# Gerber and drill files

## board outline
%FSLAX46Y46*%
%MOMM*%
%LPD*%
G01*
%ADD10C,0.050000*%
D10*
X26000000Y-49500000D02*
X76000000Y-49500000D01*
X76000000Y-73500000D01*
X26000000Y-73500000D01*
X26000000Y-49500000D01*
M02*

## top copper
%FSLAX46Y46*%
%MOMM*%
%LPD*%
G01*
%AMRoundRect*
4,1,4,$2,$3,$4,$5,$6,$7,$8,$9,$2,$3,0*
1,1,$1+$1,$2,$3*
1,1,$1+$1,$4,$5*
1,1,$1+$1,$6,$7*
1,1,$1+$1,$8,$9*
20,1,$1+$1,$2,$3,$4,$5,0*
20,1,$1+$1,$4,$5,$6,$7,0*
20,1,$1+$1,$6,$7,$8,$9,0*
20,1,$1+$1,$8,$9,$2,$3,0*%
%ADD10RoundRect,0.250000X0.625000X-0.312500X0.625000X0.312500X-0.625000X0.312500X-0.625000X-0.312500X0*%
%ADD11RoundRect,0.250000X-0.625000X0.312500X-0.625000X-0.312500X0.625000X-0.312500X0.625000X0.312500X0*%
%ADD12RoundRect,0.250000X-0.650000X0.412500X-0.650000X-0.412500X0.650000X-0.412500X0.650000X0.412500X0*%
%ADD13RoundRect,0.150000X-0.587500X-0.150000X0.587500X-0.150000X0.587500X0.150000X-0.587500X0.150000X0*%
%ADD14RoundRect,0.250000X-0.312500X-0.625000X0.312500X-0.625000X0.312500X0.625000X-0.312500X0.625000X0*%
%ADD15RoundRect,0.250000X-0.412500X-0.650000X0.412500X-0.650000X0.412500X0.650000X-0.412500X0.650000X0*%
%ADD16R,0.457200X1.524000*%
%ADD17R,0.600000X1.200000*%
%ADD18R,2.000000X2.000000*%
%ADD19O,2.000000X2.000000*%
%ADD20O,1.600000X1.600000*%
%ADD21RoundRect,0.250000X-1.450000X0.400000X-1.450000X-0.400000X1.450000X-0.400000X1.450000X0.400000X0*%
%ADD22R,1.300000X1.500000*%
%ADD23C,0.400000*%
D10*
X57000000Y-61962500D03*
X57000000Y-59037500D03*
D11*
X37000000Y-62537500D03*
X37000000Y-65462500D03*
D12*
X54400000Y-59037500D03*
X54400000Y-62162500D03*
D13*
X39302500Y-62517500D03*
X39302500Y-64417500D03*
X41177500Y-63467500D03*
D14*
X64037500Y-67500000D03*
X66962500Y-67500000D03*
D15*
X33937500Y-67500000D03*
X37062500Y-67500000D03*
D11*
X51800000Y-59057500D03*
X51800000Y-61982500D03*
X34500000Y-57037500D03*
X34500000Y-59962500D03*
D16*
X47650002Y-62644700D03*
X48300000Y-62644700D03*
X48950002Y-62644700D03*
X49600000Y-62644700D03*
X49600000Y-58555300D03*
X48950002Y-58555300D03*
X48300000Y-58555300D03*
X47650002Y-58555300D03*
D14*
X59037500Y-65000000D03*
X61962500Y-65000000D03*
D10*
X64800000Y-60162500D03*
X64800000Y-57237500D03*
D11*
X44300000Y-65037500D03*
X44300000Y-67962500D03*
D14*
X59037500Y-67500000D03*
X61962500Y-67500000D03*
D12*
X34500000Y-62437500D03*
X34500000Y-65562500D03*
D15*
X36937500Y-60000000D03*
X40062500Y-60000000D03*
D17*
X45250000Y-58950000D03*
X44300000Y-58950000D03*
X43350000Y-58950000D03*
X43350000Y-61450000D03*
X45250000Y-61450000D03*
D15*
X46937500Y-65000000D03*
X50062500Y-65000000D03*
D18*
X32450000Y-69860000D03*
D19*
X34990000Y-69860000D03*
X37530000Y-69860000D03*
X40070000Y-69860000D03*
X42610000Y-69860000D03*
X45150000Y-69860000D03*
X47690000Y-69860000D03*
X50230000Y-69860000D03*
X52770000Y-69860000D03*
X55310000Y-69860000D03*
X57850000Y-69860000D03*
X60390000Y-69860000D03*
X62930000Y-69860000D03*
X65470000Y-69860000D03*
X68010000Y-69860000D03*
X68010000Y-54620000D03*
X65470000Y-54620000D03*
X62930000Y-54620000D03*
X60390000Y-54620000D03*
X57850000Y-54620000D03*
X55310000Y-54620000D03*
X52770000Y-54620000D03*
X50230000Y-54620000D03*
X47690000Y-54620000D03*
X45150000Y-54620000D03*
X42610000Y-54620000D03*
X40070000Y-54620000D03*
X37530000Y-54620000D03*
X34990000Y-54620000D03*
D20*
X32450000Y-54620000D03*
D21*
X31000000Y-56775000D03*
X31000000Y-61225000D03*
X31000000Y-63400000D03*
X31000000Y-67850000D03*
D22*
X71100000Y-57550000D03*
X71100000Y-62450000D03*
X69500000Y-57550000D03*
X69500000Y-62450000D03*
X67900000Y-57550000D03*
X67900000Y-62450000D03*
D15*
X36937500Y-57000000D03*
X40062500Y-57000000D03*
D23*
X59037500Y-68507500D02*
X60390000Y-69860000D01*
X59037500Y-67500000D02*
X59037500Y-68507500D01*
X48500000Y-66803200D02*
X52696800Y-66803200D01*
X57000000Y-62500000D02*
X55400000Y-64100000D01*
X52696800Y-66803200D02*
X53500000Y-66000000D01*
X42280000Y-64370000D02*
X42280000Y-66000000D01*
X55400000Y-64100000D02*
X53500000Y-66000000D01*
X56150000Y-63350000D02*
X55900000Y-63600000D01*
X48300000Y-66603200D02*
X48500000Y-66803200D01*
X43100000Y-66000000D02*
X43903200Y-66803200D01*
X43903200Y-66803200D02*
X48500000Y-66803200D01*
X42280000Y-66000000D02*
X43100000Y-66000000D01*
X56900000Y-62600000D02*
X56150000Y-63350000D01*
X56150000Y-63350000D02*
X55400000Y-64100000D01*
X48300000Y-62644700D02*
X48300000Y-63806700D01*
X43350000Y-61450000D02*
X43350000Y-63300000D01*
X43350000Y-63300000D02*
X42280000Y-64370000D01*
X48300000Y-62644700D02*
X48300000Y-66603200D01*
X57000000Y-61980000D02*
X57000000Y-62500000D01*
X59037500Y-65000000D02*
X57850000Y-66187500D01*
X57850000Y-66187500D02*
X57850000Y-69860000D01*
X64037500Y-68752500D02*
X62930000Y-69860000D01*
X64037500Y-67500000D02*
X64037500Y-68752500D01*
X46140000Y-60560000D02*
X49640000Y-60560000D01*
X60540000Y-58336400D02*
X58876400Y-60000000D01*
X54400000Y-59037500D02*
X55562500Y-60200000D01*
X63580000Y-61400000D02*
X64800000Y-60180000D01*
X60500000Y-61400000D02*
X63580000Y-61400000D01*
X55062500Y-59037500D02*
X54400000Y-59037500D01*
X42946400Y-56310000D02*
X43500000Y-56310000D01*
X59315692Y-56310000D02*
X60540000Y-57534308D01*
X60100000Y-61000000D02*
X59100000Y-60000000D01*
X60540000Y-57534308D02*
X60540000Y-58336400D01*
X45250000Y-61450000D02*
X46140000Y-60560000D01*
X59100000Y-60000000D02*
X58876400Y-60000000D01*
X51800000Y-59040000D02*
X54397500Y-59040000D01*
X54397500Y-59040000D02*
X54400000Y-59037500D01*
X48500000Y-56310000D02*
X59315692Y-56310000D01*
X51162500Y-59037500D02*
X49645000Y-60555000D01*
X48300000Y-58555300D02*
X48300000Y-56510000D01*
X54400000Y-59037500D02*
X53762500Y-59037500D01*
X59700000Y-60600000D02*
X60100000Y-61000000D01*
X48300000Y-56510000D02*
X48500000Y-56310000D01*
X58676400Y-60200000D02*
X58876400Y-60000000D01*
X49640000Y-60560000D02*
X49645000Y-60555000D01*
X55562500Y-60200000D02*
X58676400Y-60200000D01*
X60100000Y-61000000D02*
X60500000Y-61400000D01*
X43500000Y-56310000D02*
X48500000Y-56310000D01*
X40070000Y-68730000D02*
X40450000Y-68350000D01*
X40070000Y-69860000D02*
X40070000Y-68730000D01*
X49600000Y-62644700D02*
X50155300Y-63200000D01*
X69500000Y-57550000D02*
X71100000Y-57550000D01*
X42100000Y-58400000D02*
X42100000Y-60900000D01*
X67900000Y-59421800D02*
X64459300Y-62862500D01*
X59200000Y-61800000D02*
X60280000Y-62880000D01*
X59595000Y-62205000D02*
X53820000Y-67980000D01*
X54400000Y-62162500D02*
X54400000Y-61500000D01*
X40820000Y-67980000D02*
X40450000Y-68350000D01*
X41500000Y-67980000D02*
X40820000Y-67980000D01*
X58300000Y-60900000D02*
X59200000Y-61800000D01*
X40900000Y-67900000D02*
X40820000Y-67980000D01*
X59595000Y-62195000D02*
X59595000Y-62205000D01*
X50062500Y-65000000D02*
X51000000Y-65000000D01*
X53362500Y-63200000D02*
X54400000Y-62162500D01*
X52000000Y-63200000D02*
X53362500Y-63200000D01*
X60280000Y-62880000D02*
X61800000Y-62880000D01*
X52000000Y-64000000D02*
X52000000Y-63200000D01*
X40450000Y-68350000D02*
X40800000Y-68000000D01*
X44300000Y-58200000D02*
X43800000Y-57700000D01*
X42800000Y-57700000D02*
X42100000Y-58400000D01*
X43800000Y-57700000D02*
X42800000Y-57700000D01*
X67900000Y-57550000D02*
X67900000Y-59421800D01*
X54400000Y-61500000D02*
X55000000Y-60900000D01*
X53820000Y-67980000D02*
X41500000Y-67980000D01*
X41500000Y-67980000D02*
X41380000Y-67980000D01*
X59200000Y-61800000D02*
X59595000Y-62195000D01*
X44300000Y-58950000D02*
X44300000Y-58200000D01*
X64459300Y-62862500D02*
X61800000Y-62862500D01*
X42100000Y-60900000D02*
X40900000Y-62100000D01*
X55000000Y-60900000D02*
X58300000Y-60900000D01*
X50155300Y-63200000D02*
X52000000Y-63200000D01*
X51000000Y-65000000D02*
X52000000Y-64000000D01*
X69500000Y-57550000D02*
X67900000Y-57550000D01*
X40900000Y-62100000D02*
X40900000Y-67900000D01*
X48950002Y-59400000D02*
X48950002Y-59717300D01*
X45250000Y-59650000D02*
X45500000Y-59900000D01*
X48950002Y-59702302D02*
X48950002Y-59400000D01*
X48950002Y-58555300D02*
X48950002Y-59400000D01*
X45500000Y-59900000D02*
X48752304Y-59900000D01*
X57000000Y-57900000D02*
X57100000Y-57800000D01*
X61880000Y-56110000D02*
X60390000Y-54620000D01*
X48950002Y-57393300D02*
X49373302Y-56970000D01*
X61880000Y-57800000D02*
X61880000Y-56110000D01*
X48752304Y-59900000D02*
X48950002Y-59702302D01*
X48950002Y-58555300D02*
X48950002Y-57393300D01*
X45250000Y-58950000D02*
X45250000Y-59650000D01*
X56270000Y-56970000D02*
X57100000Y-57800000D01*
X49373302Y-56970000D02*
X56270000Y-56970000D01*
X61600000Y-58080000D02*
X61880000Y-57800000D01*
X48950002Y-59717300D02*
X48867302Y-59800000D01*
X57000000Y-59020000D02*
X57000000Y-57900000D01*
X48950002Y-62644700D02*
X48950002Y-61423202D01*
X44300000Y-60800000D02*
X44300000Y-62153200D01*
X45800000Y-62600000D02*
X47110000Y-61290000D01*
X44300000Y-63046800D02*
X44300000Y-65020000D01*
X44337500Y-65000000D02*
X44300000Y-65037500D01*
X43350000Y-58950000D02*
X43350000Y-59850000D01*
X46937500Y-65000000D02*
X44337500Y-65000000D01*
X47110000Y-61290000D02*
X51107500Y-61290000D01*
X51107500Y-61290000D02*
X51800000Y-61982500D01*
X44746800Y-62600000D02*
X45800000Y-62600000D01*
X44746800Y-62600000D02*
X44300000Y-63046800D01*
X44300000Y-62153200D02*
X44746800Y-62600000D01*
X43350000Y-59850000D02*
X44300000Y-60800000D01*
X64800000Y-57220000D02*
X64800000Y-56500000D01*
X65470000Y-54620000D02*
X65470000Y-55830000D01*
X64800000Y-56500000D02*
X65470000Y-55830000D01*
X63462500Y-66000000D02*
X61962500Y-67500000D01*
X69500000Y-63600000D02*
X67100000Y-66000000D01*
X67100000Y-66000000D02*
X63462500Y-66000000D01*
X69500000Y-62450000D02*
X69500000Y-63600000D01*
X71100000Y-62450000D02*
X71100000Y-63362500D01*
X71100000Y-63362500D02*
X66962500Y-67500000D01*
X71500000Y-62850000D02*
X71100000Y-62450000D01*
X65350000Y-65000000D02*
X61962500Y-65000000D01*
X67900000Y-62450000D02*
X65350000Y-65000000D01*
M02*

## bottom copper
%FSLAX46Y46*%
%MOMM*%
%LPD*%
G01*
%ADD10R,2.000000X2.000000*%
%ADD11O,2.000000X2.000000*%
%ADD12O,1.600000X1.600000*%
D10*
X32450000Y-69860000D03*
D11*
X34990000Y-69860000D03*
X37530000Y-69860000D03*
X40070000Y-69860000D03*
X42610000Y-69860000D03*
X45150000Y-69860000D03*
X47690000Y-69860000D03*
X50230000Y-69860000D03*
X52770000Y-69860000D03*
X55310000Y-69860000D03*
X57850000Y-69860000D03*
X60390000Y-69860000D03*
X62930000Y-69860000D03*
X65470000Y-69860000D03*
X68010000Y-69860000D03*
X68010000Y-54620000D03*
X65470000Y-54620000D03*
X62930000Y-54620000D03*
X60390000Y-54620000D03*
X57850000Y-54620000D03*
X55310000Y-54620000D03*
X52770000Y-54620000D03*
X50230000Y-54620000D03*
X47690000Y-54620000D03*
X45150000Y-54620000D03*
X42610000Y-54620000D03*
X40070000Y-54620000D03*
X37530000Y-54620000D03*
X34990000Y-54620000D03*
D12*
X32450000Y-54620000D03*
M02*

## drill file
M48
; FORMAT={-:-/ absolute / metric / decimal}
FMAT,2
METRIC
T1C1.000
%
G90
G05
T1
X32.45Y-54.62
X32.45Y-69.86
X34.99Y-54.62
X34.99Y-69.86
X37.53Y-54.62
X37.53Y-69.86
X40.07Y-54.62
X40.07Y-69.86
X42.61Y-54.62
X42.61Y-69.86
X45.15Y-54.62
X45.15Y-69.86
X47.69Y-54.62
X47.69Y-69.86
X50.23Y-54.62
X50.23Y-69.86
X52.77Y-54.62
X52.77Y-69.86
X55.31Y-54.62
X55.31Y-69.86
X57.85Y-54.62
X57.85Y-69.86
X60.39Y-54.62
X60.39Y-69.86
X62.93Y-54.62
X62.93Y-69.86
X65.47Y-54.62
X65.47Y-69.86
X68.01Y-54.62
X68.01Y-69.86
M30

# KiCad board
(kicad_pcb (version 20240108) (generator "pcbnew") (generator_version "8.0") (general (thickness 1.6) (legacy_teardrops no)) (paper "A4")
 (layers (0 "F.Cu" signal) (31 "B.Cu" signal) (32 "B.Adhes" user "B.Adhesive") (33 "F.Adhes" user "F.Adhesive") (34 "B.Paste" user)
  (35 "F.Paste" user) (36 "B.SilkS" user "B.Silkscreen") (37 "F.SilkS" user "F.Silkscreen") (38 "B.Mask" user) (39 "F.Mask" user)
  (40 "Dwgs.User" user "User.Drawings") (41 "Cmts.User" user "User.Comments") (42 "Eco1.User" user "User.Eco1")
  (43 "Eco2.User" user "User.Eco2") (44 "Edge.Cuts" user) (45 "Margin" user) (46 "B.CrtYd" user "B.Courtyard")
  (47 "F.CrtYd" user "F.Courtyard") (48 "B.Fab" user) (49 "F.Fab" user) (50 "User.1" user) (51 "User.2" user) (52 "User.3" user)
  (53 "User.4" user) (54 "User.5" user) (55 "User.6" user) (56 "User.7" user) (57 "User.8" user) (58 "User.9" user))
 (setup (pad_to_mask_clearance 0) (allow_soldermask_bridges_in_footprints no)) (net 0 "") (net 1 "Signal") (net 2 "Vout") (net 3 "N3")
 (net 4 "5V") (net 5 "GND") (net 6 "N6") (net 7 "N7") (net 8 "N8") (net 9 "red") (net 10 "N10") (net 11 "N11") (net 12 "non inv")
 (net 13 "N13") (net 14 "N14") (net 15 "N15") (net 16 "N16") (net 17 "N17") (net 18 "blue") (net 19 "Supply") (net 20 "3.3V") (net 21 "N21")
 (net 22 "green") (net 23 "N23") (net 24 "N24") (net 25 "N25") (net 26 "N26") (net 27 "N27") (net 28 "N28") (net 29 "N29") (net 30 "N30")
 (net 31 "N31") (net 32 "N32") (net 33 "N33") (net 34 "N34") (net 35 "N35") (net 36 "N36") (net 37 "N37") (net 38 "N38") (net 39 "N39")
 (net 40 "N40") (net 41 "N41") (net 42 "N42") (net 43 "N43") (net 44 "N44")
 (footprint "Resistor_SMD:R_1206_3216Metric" (layer "F.Cu") (at 57 60.5 90)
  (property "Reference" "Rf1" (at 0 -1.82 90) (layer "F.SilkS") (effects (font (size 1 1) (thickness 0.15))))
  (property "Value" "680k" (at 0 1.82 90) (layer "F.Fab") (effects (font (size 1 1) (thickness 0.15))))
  (pad "1" smd roundrect (at -1.4625 0 90) (size 1.125 1.75) (layers "F.Cu" "F.Paste" "F.Mask") (roundrect_rratio 0.222222) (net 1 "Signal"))
  (pad "2" smd roundrect (at 1.4625 0 90) (size 1.125 1.75) (layers "F.Cu" "F.Paste" "F.Mask") (roundrect_rratio 0.222222) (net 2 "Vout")))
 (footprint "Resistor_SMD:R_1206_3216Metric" (layer "F.Cu") (at 37 64 -90)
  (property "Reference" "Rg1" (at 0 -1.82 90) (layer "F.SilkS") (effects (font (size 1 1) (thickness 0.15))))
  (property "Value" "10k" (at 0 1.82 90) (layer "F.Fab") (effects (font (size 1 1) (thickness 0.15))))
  (pad "1" smd roundrect (at -1.4625 0 270) (size 1.125 1.75) (layers "F.Cu" "F.Paste" "F.Mask") (roundrect_rratio 0.222222) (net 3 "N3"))
  (pad "2" smd roundrect (at 1.4625 0 270) (size 1.125 1.75) (layers "F.Cu" "F.Paste" "F.Mask") (roundrect_rratio 0.222222) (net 1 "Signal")))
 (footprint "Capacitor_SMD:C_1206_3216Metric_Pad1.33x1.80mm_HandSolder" (layer "F.Cu") (at 54.4 60.6 -90)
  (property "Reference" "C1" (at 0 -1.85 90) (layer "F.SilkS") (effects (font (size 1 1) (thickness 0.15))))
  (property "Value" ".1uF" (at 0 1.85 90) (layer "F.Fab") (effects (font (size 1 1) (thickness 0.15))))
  (pad "1" smd roundrect (at -1.5625 0 270) (size 1.325 1.8) (layers "F.Cu" "F.Paste" "F.Mask") (roundrect_rratio 0.188679) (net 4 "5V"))
  (pad "2" smd roundrect (at 1.5625 0 270) (size 1.325 1.8) (layers "F.Cu" "F.Paste" "F.Mask") (roundrect_rratio 0.188679) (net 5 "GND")))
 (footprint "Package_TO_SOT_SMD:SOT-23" (layer "F.Cu") (at 40.24 63.4675)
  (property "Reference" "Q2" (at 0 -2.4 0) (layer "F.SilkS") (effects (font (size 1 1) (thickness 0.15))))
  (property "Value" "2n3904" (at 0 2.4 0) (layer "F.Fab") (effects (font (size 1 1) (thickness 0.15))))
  (pad "1" smd roundrect (at -0.9375 -0.95) (size 1.475 0.6) (layers "F.Cu" "F.Paste" "F.Mask") (roundrect_rratio 0.25) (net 5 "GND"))
  (pad "2" smd roundrect (at -0.9375 0.95) (size 1.475 0.6) (layers "F.Cu" "F.Paste" "F.Mask") (roundrect_rratio 0.25) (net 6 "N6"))
  (pad "3" smd roundrect (at 0.9375 0) (size 1.475 0.6) (layers "F.Cu" "F.Paste" "F.Mask") (roundrect_rratio 0.25) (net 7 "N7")))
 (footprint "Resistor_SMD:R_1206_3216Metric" (layer "F.Cu") (at 65.5 67.5)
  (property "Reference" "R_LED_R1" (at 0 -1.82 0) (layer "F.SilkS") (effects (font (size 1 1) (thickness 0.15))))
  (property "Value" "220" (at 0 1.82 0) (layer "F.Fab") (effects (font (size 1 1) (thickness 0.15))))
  (pad "1" smd roundrect (at -1.4625 0) (size 1.125 1.75) (layers "F.Cu" "F.Paste" "F.Mask") (roundrect_rratio 0.222222) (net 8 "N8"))
  (pad "2" smd roundrect (at 1.4625 0) (size 1.125 1.75) (layers "F.Cu" "F.Paste" "F.Mask") (roundrect_rratio 0.222222) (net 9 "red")))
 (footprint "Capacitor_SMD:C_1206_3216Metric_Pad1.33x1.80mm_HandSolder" (layer "F.Cu") (at 35.5 67.5)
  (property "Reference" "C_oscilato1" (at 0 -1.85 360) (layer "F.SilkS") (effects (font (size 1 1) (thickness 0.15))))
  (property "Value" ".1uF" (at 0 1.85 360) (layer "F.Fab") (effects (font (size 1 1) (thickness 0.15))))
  (pad "1" smd roundrect (at -1.5625 0) (size 1.325 1.8) (layers "F.Cu" "F.Paste" "F.Mask") (roundrect_rratio 0.188679) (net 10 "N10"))
  (pad "2" smd roundrect (at 1.5625 0) (size 1.325 1.8) (layers "F.Cu" "F.Paste" "F.Mask") (roundrect_rratio 0.188679) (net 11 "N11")))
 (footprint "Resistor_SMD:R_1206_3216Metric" (layer "F.Cu") (at 51.8 60.52 -90)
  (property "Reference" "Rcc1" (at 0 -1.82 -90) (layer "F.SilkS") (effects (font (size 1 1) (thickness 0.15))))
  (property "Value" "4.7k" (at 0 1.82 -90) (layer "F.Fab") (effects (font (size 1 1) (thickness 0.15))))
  (pad "1" smd roundrect (at -1.4625 0 270) (size 1.125 1.75) (layers "F.Cu" "F.Paste" "F.Mask") (roundrect_rratio 0.222222) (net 4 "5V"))
  (pad "2" smd roundrect (at 1.4625 0 270) (size 1.125 1.75) (layers "F.Cu" "F.Paste" "F.Mask") (roundrect_rratio 0.222222)
   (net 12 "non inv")))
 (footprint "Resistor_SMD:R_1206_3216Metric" (layer "F.Cu") (at 34.5 58.5 -90)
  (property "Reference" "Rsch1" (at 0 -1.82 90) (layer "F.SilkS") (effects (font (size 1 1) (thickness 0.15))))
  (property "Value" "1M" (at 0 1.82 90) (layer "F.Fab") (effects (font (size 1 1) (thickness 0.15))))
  (pad "1" smd roundrect (at -1.4625 0 270) (size 1.125 1.75) (layers "F.Cu" "F.Paste" "F.Mask") (roundrect_rratio 0.222222) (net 6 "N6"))
  (pad "2" smd roundrect (at 1.4625 0 270) (size 1.125 1.75) (layers "F.Cu" "F.Paste" "F.Mask") (roundrect_rratio 0.222222) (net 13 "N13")))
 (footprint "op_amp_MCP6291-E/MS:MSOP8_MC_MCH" (layer "F.Cu") (at 48.625001 60.6 90)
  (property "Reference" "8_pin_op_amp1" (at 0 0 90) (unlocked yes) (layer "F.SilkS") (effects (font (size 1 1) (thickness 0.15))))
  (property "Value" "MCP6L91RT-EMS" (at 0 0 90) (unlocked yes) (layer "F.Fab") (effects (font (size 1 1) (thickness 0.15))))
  (pad "1" smd rect (at -2.0447 -0.974999 90) (size 1.524 0.4572) (layers "F.Cu" "F.Paste" "F.Mask") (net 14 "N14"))
  (pad "2" smd rect (at -2.0447 -0.325001 90) (size 1.524 0.4572) (layers "F.Cu" "F.Paste" "F.Mask") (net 1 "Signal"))
  (pad "3" smd rect (at -2.0447 0.325001 90) (size 1.524 0.4572) (layers "F.Cu" "F.Paste" "F.Mask") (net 12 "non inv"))
  (pad "4" smd rect (at -2.0447 0.974999 90) (size 1.524 0.4572) (layers "F.Cu" "F.Paste" "F.Mask") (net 5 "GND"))
  (pad "5" smd rect (at 2.0447 0.974999 90) (size 1.524 0.4572) (layers "F.Cu" "F.Paste" "F.Mask") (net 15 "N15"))
  (pad "6" smd rect (at 2.0447 0.325001 90) (size 1.524 0.4572) (layers "F.Cu" "F.Paste" "F.Mask") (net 2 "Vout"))
  (pad "7" smd rect (at 2.0447 -0.325001 90) (size 1.524 0.4572) (layers "F.Cu" "F.Paste" "F.Mask") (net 4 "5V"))
  (pad "8" smd rect (at 2.0447 -0.974999 90) (size 1.524 0.4572) (layers "F.Cu" "F.Paste" "F.Mask") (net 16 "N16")))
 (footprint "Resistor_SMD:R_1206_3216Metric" (layer "F.Cu") (at 60.5 65)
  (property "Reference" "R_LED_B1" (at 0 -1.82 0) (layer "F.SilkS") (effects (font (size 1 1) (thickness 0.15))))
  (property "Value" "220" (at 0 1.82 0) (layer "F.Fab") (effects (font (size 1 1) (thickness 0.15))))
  (pad "1" smd roundrect (at -1.4625 0) (size 1.125 1.75) (layers "F.Cu" "F.Paste" "F.Mask") (roundrect_rratio 0.222222) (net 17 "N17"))
  (pad "2" smd roundrect (at 1.4625 0) (size 1.125 1.75) (layers "F.Cu" "F.Paste" "F.Mask") (roundrect_rratio 0.222222) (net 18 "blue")))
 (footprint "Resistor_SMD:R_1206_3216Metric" (layer "F.Cu") (at 64.8 58.7 90)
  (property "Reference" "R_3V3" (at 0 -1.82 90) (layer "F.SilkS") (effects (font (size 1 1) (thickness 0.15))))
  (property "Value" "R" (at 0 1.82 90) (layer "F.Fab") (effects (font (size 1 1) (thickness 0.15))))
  (pad "1" smd roundrect (at -1.4625 0 90) (size 1.125 1.75) (layers "F.Cu" "F.Paste" "F.Mask") (roundrect_rratio 0.222222)
   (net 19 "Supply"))
  (pad "2" smd roundrect (at 1.4625 0 90) (size 1.125 1.75) (layers "F.Cu" "F.Paste" "F.Mask") (roundrect_rratio 0.222222) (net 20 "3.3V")))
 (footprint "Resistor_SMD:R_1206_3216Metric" (layer "F.Cu") (at 44.3 66.5 -90)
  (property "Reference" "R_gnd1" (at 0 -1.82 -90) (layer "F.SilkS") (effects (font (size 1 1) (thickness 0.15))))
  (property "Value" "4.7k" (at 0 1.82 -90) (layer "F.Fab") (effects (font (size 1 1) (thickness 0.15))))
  (pad "1" smd roundrect (at -1.4625 0 270) (size 1.125 1.75) (layers "F.Cu" "F.Paste" "F.Mask") (roundrect_rratio 0.222222)
   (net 12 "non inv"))
  (pad "2" smd roundrect (at 1.4625 0 270) (size 1.125 1.75) (layers "F.Cu" "F.Paste" "F.Mask") (roundrect_rratio 0.222222) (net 5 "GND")))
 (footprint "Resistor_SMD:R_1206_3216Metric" (layer "F.Cu") (at 60.5 67.5)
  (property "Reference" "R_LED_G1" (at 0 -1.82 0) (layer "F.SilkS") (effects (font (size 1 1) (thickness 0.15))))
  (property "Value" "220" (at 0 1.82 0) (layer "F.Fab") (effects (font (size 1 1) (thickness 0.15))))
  (pad "1" smd roundrect (at -1.4625 0) (size 1.125 1.75) (layers "F.Cu" "F.Paste" "F.Mask") (roundrect_rratio 0.222222) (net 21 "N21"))
  (pad "2" smd roundrect (at 1.4625 0) (size 1.125 1.75) (layers "F.Cu" "F.Paste" "F.Mask") (roundrect_rratio 0.222222) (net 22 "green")))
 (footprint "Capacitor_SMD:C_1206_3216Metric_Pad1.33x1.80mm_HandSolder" (layer "F.Cu") (at 34.5 64 -90)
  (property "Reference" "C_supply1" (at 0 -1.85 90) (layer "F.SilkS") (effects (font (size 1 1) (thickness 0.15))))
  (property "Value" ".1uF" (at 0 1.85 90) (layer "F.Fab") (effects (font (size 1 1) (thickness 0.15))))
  (pad "1" smd roundrect (at -1.5625 0 270) (size 1.325 1.8) (layers "F.Cu" "F.Paste" "F.Mask") (roundrect_rratio 0.188679) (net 13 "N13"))
  (pad "2" smd roundrect (at 1.5625 0 270) (size 1.325 1.8) (layers "F.Cu" "F.Paste" "F.Mask") (roundrect_rratio 0.188679) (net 5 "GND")))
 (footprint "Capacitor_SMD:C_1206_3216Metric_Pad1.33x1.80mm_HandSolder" (layer "F.Cu") (at 38.5 60)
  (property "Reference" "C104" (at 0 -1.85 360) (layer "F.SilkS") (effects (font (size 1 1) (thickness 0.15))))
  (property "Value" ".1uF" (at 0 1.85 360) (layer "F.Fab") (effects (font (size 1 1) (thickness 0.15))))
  (pad "1" smd roundrect (at -1.5625 0) (size 1.325 1.8) (layers "F.Cu" "F.Paste" "F.Mask") (roundrect_rratio 0.188679) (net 6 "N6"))
  (pad "2" smd roundrect (at 1.5625 0) (size 1.325 1.8) (layers "F.Cu" "F.Paste" "F.Mask") (roundrect_rratio 0.188679) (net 3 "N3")))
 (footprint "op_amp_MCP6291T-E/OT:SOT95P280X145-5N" (layer "F.Cu") (at 44.3 60.2 -90)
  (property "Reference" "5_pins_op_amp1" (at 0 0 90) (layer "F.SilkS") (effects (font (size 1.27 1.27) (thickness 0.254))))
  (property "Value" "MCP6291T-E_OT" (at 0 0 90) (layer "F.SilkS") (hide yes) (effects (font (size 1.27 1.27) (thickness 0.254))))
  (pad "1" smd rect (at -1.25 -0.95) (size 0.6 1.2) (layers "F.Cu" "F.Paste" "F.Mask") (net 2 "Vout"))
  (pad "2" smd rect (at -1.25 0) (size 0.6 1.2) (layers "F.Cu" "F.Paste" "F.Mask") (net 5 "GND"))
  (pad "3" smd rect (at -1.25 0.95) (size 0.6 1.2) (layers "F.Cu" "F.Paste" "F.Mask") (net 12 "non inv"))
  (pad "4" smd rect (at 1.25 0.95) (size 0.6 1.2) (layers "F.Cu" "F.Paste" "F.Mask") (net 1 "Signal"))
  (pad "5" smd rect (at 1.25 -0.95) (size 0.6 1.2) (layers "F.Cu" "F.Paste" "F.Mask") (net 4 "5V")))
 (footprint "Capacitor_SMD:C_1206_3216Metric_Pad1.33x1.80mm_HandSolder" (layer "F.Cu") (at 48.5 65)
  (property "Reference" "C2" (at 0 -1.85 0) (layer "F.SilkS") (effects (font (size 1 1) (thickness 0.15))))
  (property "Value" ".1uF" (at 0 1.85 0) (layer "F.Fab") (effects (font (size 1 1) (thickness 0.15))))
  (pad "1" smd roundrect (at -1.5625 0) (size 1.325 1.8) (layers "F.Cu" "F.Paste" "F.Mask") (roundrect_rratio 0.188679) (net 12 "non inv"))
  (pad "2" smd roundrect (at 1.5625 0) (size 1.325 1.8) (layers "F.Cu" "F.Paste" "F.Mask") (roundrect_rratio 0.188679) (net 5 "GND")))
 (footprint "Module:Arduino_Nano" (layer "F.Cu") (at 32.45 69.86 90)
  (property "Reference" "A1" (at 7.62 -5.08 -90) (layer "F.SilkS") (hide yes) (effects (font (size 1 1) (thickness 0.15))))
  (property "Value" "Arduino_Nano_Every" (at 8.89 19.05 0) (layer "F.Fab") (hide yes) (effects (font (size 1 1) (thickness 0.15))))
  (pad "1" thru_hole rect (at 0 0 90) (size 2 2) (drill 1) (layers "*.Cu" "*.Mask") (remove_unused_layers no) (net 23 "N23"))
  (pad "2" thru_hole oval (at 0 2.54 90) (size 2 2) (drill 1) (layers "*.Cu" "*.Mask") (remove_unused_layers no) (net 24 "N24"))
  (pad "3" thru_hole oval (at 0 5.08 90) (size 2 2) (drill 1) (layers "*.Cu" "*.Mask") (remove_unused_layers no) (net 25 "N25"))
  (pad "4" thru_hole oval (at 0 7.62 90) (size 2 2) (drill 1) (layers "*.Cu" "*.Mask") (remove_unused_layers no) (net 5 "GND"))
  (pad "5" thru_hole oval (at 0 10.16 90) (size 2 2) (drill 1) (layers "*.Cu" "*.Mask") (remove_unused_layers no) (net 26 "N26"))
  (pad "6" thru_hole oval (at 0 12.7 90) (size 2 2) (drill 1) (layers "*.Cu" "*.Mask") (remove_unused_layers no) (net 11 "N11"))
  (pad "7" thru_hole oval (at 0 15.24 90) (size 2 2) (drill 1) (layers "*.Cu" "*.Mask") (remove_unused_layers no) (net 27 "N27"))
  (pad "8" thru_hole oval (at 0 17.78 90) (size 2 2) (drill 1) (layers "*.Cu" "*.Mask") (remove_unused_layers no) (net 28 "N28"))
  (pad "9" thru_hole oval (at 0 20.32 90) (size 2 2) (drill 1) (layers "*.Cu" "*.Mask") (remove_unused_layers no) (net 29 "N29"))
  (pad "10" thru_hole oval (at 0 22.86 90) (size 2 2) (drill 1) (layers "*.Cu" "*.Mask") (remove_unused_layers no) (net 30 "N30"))
  (pad "11" thru_hole oval (at 0 25.4 90) (size 2 2) (drill 1) (layers "*.Cu" "*.Mask") (remove_unused_layers no) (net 17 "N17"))
  (pad "12" thru_hole oval (at 0 27.94 90) (size 2 2) (drill 1) (layers "*.Cu" "*.Mask") (remove_unused_layers no) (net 21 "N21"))
  (pad "13" thru_hole oval (at 0 30.48 90) (size 2 2) (drill 1) (layers "*.Cu" "*.Mask") (remove_unused_layers no) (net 8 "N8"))
  (pad "14" thru_hole oval (at 0 33.02 90) (size 2 2) (drill 1) (layers "*.Cu" "*.Mask") (remove_unused_layers no) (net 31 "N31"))
  (pad "15" thru_hole oval (at 0 35.56 90) (size 2 2) (drill 1) (layers "*.Cu" "*.Mask") (remove_unused_layers no) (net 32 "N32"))
  (pad "16" thru_hole oval (at 15.24 35.56 90) (size 2 2) (drill 1) (layers "*.Cu" "*.Mask") (remove_unused_layers no) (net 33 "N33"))
  (pad "17" thru_hole oval (at 15.24 33.02 90) (size 2 2) (drill 1) (layers "*.Cu" "*.Mask") (remove_unused_layers no) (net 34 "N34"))
  (pad "18" thru_hole oval (at 15.24 30.48 90) (size 2 2) (drill 1) (layers "*.Cu" "*.Mask") (remove_unused_layers no) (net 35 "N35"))
  (pad "19" thru_hole oval (at 15.24 27.94 90) (size 2 2) (drill 1) (layers "*.Cu" "*.Mask") (remove_unused_layers no) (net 2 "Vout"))
  (pad "20" thru_hole oval (at 15.24 25.4 90) (size 2 2) (drill 1) (layers "*.Cu" "*.Mask") (remove_unused_layers no) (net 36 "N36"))
  (pad "21" thru_hole oval (at 15.24 22.86 90) (size 2 2) (drill 1) (layers "*.Cu" "*.Mask") (remove_unused_layers no) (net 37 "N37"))
  (pad "22" thru_hole oval (at 15.24 20.32 90) (size 2 2) (drill 1) (layers "*.Cu" "*.Mask" "Eco2.User") (remove_unused_layers no)
   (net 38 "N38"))
  (pad "23" thru_hole oval (at 15.24 17.78 90) (size 2 2) (drill 1) (layers "*.Cu" "*.Mask") (remove_unused_layers no) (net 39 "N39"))
  (pad "24" thru_hole oval (at 15.24 15.24 90) (size 2 2) (drill 1) (layers "*.Cu" "*.Mask") (remove_unused_layers no) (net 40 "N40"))
  (pad "25" thru_hole oval (at 15.24 12.7 90) (size 2 2) (drill 1) (layers "*.Cu" "*.Mask" "B.SilkS") (remove_unused_layers no)
   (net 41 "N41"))
  (pad "26" thru_hole oval (at 15.24 10.16 90) (size 2 2) (drill 1) (layers "*.Cu" "*.Mask") (remove_unused_layers no) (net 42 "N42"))
  (pad "27" thru_hole oval (at 15.24 7.62 90) (size 2 2) (drill 1) (layers "*.Cu" "*.Mask") (remove_unused_layers no) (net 4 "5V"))
  (pad "28" thru_hole oval (at 15.24 5.08 90) (size 2 2) (drill 1) (layers "*.Cu" "*.Mask") (remove_unused_layers no) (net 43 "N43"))
  (pad "29" thru_hole oval (at 15.24 2.54 90) (size 2 2) (drill 1) (layers "*.Cu" "*.Mask") (remove_unused_layers no) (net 5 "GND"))
  (pad "30" thru_hole oval (at 15.24 0 90) (size 1.6 1.6) (drill 1) (layers "*.Cu" "*.Mask") (remove_unused_layers no) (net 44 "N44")))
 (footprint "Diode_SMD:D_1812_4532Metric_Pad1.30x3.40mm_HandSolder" (layer "F.Cu") (at 31 59 -90)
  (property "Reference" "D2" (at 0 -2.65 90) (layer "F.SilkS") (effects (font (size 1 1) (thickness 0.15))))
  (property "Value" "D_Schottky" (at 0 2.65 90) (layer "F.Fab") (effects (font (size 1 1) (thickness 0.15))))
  (pad "1" smd roundrect (at -2.225 0 270) (size 1.3 3.4) (layers "F.Cu" "F.Paste" "F.Mask") (roundrect_rratio 0.192308) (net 13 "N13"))
  (pad "2" smd roundrect (at 2.225 0 270) (size 1.3 3.4) (layers "F.Cu" "F.Paste" "F.Mask") (roundrect_rratio 0.192308) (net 10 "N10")))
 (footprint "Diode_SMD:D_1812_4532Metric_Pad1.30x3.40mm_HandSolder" (layer "F.Cu") (at 31 65.625 -90)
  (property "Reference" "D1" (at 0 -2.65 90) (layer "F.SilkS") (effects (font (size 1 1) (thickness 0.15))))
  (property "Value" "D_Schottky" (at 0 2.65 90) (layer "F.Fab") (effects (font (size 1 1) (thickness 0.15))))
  (pad "1" smd roundrect (at -2.225 0 270) (size 1.3 3.4) (layers "F.Cu" "F.Paste" "F.Mask") (roundrect_rratio 0.192308) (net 10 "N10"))
  (pad "2" smd roundrect (at 2.225 0 270) (size 1.3 3.4) (layers "F.Cu" "F.Paste" "F.Mask") (roundrect_rratio 0.192308) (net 4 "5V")))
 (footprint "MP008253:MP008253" (layer "F.Cu") (at 69.5 60 -90)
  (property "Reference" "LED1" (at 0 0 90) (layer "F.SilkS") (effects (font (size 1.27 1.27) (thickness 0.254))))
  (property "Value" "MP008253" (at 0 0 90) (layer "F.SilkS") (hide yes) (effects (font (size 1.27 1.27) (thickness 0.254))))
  (pad "1" smd rect (at -2.45 -1.6) (size 1.3 1.5) (layers "F.Cu" "F.Paste" "F.Mask") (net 5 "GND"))
  (pad "2" smd rect (at 2.45 -1.6) (size 1.3 1.5) (layers "F.Cu" "F.Paste" "F.Mask") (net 9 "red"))
  (pad "3" smd rect (at -2.45 0) (size 1.3 1.5) (layers "F.Cu" "F.Paste" "F.Mask") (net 5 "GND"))
  (pad "4" smd rect (at 2.45 0) (size 1.3 1.5) (layers "F.Cu" "F.Paste" "F.Mask") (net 22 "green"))
  (pad "5" smd rect (at -2.45 1.6) (size 1.3 1.5) (layers "F.Cu" "F.Paste" "F.Mask") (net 5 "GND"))
  (pad "6" smd rect (at 2.45 1.6) (size 1.3 1.5) (layers "F.Cu" "F.Paste" "F.Mask") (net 18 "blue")))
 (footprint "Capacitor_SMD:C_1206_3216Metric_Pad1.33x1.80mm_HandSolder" (layer "F.Cu") (at 38.5 57)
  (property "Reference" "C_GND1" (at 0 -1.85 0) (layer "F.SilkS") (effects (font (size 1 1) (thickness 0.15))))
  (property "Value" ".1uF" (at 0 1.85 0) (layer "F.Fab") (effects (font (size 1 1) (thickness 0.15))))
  (pad "1" smd roundrect (at -1.5625 0) (size 1.325 1.8) (layers "F.Cu" "F.Paste" "F.Mask") (roundrect_rratio 0.188679) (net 5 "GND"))
  (pad "2" smd roundrect (at 1.5625 0) (size 1.325 1.8) (layers "F.Cu" "F.Paste" "F.Mask") (roundrect_rratio 0.188679) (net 4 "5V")))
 (gr_rect (start 26 49.5) (end 76 73.5) (stroke (width 0.05) (type default)) (fill none) (layer "Edge.Cuts"))
 (segment (start 59.0375 68.5075) (end 60.39 69.86) (width 0.4) (layer "F.Cu") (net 21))
 (segment (start 59.0375 67.5) (end 59.0375 68.5075) (width 0.4) (layer "F.Cu") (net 21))
 (segment (start 48.5 66.8032) (end 52.6968 66.8032) (width 0.4) (layer "F.Cu") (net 1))
 (segment (start 57 62.5) (end 55.4 64.1) (width 0.4) (layer "F.Cu") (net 1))
 (segment (start 52.6968 66.8032) (end 53.5 66) (width 0.4) (layer "F.Cu") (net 1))
 (segment (start 42.28 64.37) (end 42.28 66) (width 0.4) (layer "F.Cu") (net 1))
 (segment (start 55.4 64.1) (end 53.5 66) (width 0.4) (layer "F.Cu") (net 1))
 (segment (start 56.15 63.35) (end 55.9 63.6) (width 0.4) (layer "F.Cu") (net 1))
 (segment (start 48.3 66.6032) (end 48.5 66.8032) (width 0.4) (layer "F.Cu") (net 1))
 (segment (start 43.1 66) (end 43.9032 66.8032) (width 0.4) (layer "F.Cu") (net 1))
 (segment (start 43.9032 66.8032) (end 48.5 66.8032) (width 0.4) (layer "F.Cu") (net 1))
 (segment (start 42.28 66) (end 43.1 66) (width 0.4) (layer "F.Cu") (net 1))
 (segment (start 56.9 62.6) (end 56.15 63.35) (width 0.4) (layer "F.Cu") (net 1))
 (segment (start 56.15 63.35) (end 55.4 64.1) (width 0.4) (layer "F.Cu") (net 1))
 (segment (start 48.3 62.6447) (end 48.3 63.8067) (width 0.4) (layer "F.Cu") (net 1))
 (segment (start 43.35 61.45) (end 43.35 63.3) (width 0.4) (layer "F.Cu") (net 1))
 (segment (start 43.35 63.3) (end 42.28 64.37) (width 0.4) (layer "F.Cu") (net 1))
 (segment (start 48.3 62.6447) (end 48.3 66.6032) (width 0.4) (layer "F.Cu") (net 1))
 (segment (start 57 61.98) (end 57 62.5) (width 0.4) (layer "F.Cu") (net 1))
 (segment (start 59.0375 65) (end 57.85 66.1875) (width 0.4) (layer "F.Cu") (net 17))
 (segment (start 57.85 66.1875) (end 57.85 69.86) (width 0.4) (layer "F.Cu") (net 17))
 (segment (start 64.0375 68.7525) (end 62.93 69.86) (width 0.4) (layer "F.Cu") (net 8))
 (segment (start 64.0375 67.5) (end 64.0375 68.7525) (width 0.4) (layer "F.Cu") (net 8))
 (segment (start 46.14 60.56) (end 49.64 60.56) (width 0.4) (layer "F.Cu") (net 19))
 (segment (start 60.54 58.3364) (end 58.8764 60) (width 0.4) (layer "F.Cu") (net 19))
 (segment (start 54.4 59.0375) (end 55.5625 60.2) (width 0.4) (layer "F.Cu") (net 19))
 (segment (start 63.58 61.4) (end 64.8 60.18) (width 0.4) (layer "F.Cu") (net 19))
 (segment (start 60.5 61.4) (end 63.58 61.4) (width 0.4) (layer "F.Cu") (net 19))
 (segment (start 55.0625 59.0375) (end 54.4 59.0375) (width 0.4) (layer "F.Cu") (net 19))
 (segment (start 42.9464 56.31) (end 43.5 56.31) (width 0.4) (layer "F.Cu") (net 19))
 (segment (start 59.315692 56.31) (end 60.54 57.534308) (width 0.4) (layer "F.Cu") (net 19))
 (segment (start 60.1 61) (end 59.1 60) (width 0.4) (layer "F.Cu") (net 19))
 (segment (start 60.54 57.534308) (end 60.54 58.3364) (width 0.4) (layer "F.Cu") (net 19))
 (segment (start 45.25 61.45) (end 46.14 60.56) (width 0.4) (layer "F.Cu") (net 19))
 (segment (start 59.1 60) (end 58.8764 60) (width 0.4) (layer "F.Cu") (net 19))
 (segment (start 51.8 59.04) (end 54.3975 59.04) (width 0.4) (layer "F.Cu") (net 19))
 (segment (start 54.3975 59.04) (end 54.4 59.0375) (width 0.4) (layer "F.Cu") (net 19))
 (segment (start 48.5 56.31) (end 59.315692 56.31) (width 0.4) (layer "F.Cu") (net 19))
 (segment (start 51.1625 59.0375) (end 49.645 60.555) (width 0.4) (layer "F.Cu") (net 19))
 (segment (start 48.3 58.5553) (end 48.3 56.51) (width 0.4) (layer "F.Cu") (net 19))
 (segment (start 54.4 59.0375) (end 53.7625 59.0375) (width 0.4) (layer "F.Cu") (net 19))
 (segment (start 59.7 60.6) (end 60.1 61) (width 0.4) (layer "F.Cu") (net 19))
 (segment (start 48.3 56.51) (end 48.5 56.31) (width 0.4) (layer "F.Cu") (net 19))
 (segment (start 58.6764 60.2) (end 58.8764 60) (width 0.4) (layer "F.Cu") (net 19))
 (segment (start 49.64 60.56) (end 49.645 60.555) (width 0.4) (layer "F.Cu") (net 19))
 (segment (start 55.5625 60.2) (end 58.6764 60.2) (width 0.4) (layer "F.Cu") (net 19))
 (segment (start 60.1 61) (end 60.5 61.4) (width 0.4) (layer "F.Cu") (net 19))
 (segment (start 43.5 56.31) (end 48.5 56.31) (width 0.4) (layer "F.Cu") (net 19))
 (segment (start 40.07 68.73) (end 40.45 68.35) (width 0.4) (layer "F.Cu") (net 5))
 (segment (start 40.07 69.86) (end 40.07 68.73) (width 0.4) (layer "F.Cu") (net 5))
 (segment (start 49.6 62.6447) (end 50.1553 63.2) (width 0.4) (layer "F.Cu") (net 5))
 (segment (start 69.5 57.55) (end 71.1 57.55) (width 0.4) (layer "F.Cu") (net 5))
 (segment (start 42.1 58.4) (end 42.1 60.9) (width 0.4) (layer "F.Cu") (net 5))
 (segment (start 67.9 59.4218) (end 64.4593 62.8625) (width 0.4) (layer "F.Cu") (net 5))
 (segment (start 59.2 61.8) (end 60.28 62.88) (width 0.4) (layer "F.Cu") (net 5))
 (segment (start 59.595 62.205) (end 53.82 67.98) (width 0.4) (layer "F.Cu") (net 5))
 (segment (start 54.4 62.1625) (end 54.4 61.5) (width 0.4) (layer "F.Cu") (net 5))
 (segment (start 40.82 67.98) (end 40.45 68.35) (width 0.4) (layer "F.Cu") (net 5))
 (segment (start 41.5 67.98) (end 40.82 67.98) (width 0.4) (layer "F.Cu") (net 5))
 (segment (start 58.3 60.9) (end 59.2 61.8) (width 0.4) (layer "F.Cu") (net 5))
 (segment (start 40.9 67.9) (end 40.82 67.98) (width 0.4) (layer "F.Cu") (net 5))
 (segment (start 59.595 62.195) (end 59.595 62.205) (width 0.4) (layer "F.Cu") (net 5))
 (segment (start 50.0625 65) (end 51 65) (width 0.4) (layer "F.Cu") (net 5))
 (segment (start 53.3625 63.2) (end 54.4 62.1625) (width 0.4) (layer "F.Cu") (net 5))
 (segment (start 52 63.2) (end 53.3625 63.2) (width 0.4) (layer "F.Cu") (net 5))
 (segment (start 60.28 62.88) (end 61.8 62.88) (width 0.4) (layer "F.Cu") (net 5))
 (segment (start 52 64) (end 52 63.2) (width 0.4) (layer "F.Cu") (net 5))
 (segment (start 40.45 68.35) (end 40.8 68) (width 0.4) (layer "F.Cu") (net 5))
 (segment (start 44.3 58.2) (end 43.8 57.7) (width 0.4) (layer "F.Cu") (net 5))
 (segment (start 42.8 57.7) (end 42.1 58.4) (width 0.4) (layer "F.Cu") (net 5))
 (segment (start 43.8 57.7) (end 42.8 57.7) (width 0.4) (layer "F.Cu") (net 5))
 (segment (start 67.9 57.55) (end 67.9 59.4218) (width 0.4) (layer "F.Cu") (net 5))
 (segment (start 54.4 61.5) (end 55 60.9) (width 0.4) (layer "F.Cu") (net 5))
 (segment (start 53.82 67.98) (end 41.5 67.98) (width 0.4) (layer "F.Cu") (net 5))
 (segment (start 41.5 67.98) (end 41.38 67.98) (width 0.4) (layer "F.Cu") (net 5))
 (segment (start 59.2 61.8) (end 59.595 62.195) (width 0.4) (layer "F.Cu") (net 5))
 (segment (start 44.3 58.95) (end 44.3 58.2) (width 0.4) (layer "F.Cu") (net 5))
 (segment (start 64.4593 62.8625) (end 61.8 62.8625) (width 0.4) (layer "F.Cu") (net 5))
 (segment (start 42.1 60.9) (end 40.9 62.1) (width 0.4) (layer "F.Cu") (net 5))
 (segment (start 55 60.9) (end 58.3 60.9) (width 0.4) (layer "F.Cu") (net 5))
 (segment (start 50.1553 63.2) (end 52 63.2) (width 0.4) (layer "F.Cu") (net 5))
 (segment (start 51 65) (end 52 64) (width 0.4) (layer "F.Cu") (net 5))
 (segment (start 69.5 57.55) (end 67.9 57.55) (width 0.4) (layer "F.Cu") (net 5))
 (segment (start 40.9 62.1) (end 40.9 67.9) (width 0.4) (layer "F.Cu") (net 5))
 (segment (start 48.950002 59.4) (end 48.950002 59.7173) (width 0.4) (layer "F.Cu") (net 2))
 (segment (start 45.25 59.65) (end 45.5 59.9) (width 0.4) (layer "F.Cu") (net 2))
 (segment (start 48.950002 59.702302) (end 48.950002 59.4) (width 0.4) (layer "F.Cu") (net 2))
 (segment (start 48.950002 58.5553) (end 48.950002 59.4) (width 0.4) (layer "F.Cu") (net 2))
 (segment (start 45.5 59.9) (end 48.752304 59.9) (width 0.4) (layer "F.Cu") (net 2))
 (segment (start 57 57.9) (end 57.1 57.8) (width 0.4) (layer "F.Cu") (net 2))
 (segment (start 61.88 56.11) (end 60.39 54.62) (width 0.4) (layer "F.Cu") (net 2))
 (segment (start 48.950002 57.3933) (end 49.373302 56.97) (width 0.4) (layer "F.Cu") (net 2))
 (segment (start 61.88 57.8) (end 61.88 56.11) (width 0.4) (layer "F.Cu") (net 2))
 (segment (start 48.752304 59.9) (end 48.950002 59.702302) (width 0.4) (layer "F.Cu") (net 2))
 (segment (start 48.950002 58.5553) (end 48.950002 57.3933) (width 0.4) (layer "F.Cu") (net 2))
 (segment (start 45.25 58.95) (end 45.25 59.65) (width 0.4) (layer "F.Cu") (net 2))
 (segment (start 56.27 56.97) (end 57.1 57.8) (width 0.4) (layer "F.Cu") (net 2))
 (segment (start 49.373302 56.97) (end 56.27 56.97) (width 0.4) (layer "F.Cu") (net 2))
 (segment (start 61.6 58.08) (end 61.88 57.8) (width 0.4) (layer "F.Cu") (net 2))
 (segment (start 48.950002 59.7173) (end 48.867302 59.8) (width 0.4) (layer "F.Cu") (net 2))
 (segment (start 57 59.02) (end 57 57.9) (width 0.4) (layer "F.Cu") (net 2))
 (segment (start 48.950002 62.6447) (end 48.950002 61.423202) (width 0.4) (layer "F.Cu") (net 12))
 (segment (start 44.3 60.8) (end 44.3 62.1532) (width 0.4) (layer "F.Cu") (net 12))
 (segment (start 45.8 62.6) (end 47.11 61.29) (width 0.4) (layer "F.Cu") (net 12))
 (segment (start 44.3 63.0468) (end 44.3 65.02) (width 0.4) (layer "F.Cu") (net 12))
 (segment (start 44.3375 65) (end 44.3 65.0375) (width 0.4) (layer "F.Cu") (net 12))
 (segment (start 43.35 58.95) (end 43.35 59.85) (width 0.4) (layer "F.Cu") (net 12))
 (segment (start 46.9375 65) (end 44.3375 65) (width 0.4) (layer "F.Cu") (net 12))
 (segment (start 47.11 61.29) (end 51.1075 61.29) (width 0.4) (layer "F.Cu") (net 12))
 (segment (start 51.1075 61.29) (end 51.8 61.9825) (width 0.4) (layer "F.Cu") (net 12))
 (segment (start 44.7468 62.6) (end 45.8 62.6) (width 0.4) (layer "F.Cu") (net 12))
 (segment (start 44.7468 62.6) (end 44.3 63.0468) (width 0.4) (layer "F.Cu") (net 12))
 (segment (start 44.3 62.1532) (end 44.7468 62.6) (width 0.4) (layer "F.Cu") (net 12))
 (segment (start 43.35 59.85) (end 44.3 60.8) (width 0.4) (layer "F.Cu") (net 12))
 (segment (start 64.8 57.22) (end 64.8 56.5) (width 0.4) (layer "F.Cu") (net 20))
 (segment (start 65.47 54.62) (end 65.47 55.83) (width 0.4) (layer "F.Cu") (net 20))
 (segment (start 64.8 56.5) (end 65.47 55.83) (width 0.4) (layer "F.Cu") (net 20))
 (segment (start 63.4625 66) (end 61.9625 67.5) (width 0.4) (layer "F.Cu") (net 22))
 (segment (start 69.5 63.6) (end 67.1 66) (width 0.4) (layer "F.Cu") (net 22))
 (segment (start 67.1 66) (end 63.4625 66) (width 0.4) (layer "F.Cu") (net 22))
 (segment (start 69.5 62.45) (end 69.5 63.6) (width 0.4) (layer "F.Cu") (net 22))
 (segment (start 71.1 62.45) (end 71.1 63.3625) (width 0.4) (layer "F.Cu") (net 9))
 (segment (start 71.1 63.3625) (end 66.9625 67.5) (width 0.4) (layer "F.Cu") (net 9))
 (segment (start 71.5 62.85) (end 71.1 62.45) (width 0.4) (layer "F.Cu") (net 9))
 (segment (start 65.35 65) (end 61.9625 65) (width 0.4) (layer "F.Cu") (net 18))
 (segment (start 67.9 62.45) (end 65.35 65) (width 0.4) (layer "F.Cu") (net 18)))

